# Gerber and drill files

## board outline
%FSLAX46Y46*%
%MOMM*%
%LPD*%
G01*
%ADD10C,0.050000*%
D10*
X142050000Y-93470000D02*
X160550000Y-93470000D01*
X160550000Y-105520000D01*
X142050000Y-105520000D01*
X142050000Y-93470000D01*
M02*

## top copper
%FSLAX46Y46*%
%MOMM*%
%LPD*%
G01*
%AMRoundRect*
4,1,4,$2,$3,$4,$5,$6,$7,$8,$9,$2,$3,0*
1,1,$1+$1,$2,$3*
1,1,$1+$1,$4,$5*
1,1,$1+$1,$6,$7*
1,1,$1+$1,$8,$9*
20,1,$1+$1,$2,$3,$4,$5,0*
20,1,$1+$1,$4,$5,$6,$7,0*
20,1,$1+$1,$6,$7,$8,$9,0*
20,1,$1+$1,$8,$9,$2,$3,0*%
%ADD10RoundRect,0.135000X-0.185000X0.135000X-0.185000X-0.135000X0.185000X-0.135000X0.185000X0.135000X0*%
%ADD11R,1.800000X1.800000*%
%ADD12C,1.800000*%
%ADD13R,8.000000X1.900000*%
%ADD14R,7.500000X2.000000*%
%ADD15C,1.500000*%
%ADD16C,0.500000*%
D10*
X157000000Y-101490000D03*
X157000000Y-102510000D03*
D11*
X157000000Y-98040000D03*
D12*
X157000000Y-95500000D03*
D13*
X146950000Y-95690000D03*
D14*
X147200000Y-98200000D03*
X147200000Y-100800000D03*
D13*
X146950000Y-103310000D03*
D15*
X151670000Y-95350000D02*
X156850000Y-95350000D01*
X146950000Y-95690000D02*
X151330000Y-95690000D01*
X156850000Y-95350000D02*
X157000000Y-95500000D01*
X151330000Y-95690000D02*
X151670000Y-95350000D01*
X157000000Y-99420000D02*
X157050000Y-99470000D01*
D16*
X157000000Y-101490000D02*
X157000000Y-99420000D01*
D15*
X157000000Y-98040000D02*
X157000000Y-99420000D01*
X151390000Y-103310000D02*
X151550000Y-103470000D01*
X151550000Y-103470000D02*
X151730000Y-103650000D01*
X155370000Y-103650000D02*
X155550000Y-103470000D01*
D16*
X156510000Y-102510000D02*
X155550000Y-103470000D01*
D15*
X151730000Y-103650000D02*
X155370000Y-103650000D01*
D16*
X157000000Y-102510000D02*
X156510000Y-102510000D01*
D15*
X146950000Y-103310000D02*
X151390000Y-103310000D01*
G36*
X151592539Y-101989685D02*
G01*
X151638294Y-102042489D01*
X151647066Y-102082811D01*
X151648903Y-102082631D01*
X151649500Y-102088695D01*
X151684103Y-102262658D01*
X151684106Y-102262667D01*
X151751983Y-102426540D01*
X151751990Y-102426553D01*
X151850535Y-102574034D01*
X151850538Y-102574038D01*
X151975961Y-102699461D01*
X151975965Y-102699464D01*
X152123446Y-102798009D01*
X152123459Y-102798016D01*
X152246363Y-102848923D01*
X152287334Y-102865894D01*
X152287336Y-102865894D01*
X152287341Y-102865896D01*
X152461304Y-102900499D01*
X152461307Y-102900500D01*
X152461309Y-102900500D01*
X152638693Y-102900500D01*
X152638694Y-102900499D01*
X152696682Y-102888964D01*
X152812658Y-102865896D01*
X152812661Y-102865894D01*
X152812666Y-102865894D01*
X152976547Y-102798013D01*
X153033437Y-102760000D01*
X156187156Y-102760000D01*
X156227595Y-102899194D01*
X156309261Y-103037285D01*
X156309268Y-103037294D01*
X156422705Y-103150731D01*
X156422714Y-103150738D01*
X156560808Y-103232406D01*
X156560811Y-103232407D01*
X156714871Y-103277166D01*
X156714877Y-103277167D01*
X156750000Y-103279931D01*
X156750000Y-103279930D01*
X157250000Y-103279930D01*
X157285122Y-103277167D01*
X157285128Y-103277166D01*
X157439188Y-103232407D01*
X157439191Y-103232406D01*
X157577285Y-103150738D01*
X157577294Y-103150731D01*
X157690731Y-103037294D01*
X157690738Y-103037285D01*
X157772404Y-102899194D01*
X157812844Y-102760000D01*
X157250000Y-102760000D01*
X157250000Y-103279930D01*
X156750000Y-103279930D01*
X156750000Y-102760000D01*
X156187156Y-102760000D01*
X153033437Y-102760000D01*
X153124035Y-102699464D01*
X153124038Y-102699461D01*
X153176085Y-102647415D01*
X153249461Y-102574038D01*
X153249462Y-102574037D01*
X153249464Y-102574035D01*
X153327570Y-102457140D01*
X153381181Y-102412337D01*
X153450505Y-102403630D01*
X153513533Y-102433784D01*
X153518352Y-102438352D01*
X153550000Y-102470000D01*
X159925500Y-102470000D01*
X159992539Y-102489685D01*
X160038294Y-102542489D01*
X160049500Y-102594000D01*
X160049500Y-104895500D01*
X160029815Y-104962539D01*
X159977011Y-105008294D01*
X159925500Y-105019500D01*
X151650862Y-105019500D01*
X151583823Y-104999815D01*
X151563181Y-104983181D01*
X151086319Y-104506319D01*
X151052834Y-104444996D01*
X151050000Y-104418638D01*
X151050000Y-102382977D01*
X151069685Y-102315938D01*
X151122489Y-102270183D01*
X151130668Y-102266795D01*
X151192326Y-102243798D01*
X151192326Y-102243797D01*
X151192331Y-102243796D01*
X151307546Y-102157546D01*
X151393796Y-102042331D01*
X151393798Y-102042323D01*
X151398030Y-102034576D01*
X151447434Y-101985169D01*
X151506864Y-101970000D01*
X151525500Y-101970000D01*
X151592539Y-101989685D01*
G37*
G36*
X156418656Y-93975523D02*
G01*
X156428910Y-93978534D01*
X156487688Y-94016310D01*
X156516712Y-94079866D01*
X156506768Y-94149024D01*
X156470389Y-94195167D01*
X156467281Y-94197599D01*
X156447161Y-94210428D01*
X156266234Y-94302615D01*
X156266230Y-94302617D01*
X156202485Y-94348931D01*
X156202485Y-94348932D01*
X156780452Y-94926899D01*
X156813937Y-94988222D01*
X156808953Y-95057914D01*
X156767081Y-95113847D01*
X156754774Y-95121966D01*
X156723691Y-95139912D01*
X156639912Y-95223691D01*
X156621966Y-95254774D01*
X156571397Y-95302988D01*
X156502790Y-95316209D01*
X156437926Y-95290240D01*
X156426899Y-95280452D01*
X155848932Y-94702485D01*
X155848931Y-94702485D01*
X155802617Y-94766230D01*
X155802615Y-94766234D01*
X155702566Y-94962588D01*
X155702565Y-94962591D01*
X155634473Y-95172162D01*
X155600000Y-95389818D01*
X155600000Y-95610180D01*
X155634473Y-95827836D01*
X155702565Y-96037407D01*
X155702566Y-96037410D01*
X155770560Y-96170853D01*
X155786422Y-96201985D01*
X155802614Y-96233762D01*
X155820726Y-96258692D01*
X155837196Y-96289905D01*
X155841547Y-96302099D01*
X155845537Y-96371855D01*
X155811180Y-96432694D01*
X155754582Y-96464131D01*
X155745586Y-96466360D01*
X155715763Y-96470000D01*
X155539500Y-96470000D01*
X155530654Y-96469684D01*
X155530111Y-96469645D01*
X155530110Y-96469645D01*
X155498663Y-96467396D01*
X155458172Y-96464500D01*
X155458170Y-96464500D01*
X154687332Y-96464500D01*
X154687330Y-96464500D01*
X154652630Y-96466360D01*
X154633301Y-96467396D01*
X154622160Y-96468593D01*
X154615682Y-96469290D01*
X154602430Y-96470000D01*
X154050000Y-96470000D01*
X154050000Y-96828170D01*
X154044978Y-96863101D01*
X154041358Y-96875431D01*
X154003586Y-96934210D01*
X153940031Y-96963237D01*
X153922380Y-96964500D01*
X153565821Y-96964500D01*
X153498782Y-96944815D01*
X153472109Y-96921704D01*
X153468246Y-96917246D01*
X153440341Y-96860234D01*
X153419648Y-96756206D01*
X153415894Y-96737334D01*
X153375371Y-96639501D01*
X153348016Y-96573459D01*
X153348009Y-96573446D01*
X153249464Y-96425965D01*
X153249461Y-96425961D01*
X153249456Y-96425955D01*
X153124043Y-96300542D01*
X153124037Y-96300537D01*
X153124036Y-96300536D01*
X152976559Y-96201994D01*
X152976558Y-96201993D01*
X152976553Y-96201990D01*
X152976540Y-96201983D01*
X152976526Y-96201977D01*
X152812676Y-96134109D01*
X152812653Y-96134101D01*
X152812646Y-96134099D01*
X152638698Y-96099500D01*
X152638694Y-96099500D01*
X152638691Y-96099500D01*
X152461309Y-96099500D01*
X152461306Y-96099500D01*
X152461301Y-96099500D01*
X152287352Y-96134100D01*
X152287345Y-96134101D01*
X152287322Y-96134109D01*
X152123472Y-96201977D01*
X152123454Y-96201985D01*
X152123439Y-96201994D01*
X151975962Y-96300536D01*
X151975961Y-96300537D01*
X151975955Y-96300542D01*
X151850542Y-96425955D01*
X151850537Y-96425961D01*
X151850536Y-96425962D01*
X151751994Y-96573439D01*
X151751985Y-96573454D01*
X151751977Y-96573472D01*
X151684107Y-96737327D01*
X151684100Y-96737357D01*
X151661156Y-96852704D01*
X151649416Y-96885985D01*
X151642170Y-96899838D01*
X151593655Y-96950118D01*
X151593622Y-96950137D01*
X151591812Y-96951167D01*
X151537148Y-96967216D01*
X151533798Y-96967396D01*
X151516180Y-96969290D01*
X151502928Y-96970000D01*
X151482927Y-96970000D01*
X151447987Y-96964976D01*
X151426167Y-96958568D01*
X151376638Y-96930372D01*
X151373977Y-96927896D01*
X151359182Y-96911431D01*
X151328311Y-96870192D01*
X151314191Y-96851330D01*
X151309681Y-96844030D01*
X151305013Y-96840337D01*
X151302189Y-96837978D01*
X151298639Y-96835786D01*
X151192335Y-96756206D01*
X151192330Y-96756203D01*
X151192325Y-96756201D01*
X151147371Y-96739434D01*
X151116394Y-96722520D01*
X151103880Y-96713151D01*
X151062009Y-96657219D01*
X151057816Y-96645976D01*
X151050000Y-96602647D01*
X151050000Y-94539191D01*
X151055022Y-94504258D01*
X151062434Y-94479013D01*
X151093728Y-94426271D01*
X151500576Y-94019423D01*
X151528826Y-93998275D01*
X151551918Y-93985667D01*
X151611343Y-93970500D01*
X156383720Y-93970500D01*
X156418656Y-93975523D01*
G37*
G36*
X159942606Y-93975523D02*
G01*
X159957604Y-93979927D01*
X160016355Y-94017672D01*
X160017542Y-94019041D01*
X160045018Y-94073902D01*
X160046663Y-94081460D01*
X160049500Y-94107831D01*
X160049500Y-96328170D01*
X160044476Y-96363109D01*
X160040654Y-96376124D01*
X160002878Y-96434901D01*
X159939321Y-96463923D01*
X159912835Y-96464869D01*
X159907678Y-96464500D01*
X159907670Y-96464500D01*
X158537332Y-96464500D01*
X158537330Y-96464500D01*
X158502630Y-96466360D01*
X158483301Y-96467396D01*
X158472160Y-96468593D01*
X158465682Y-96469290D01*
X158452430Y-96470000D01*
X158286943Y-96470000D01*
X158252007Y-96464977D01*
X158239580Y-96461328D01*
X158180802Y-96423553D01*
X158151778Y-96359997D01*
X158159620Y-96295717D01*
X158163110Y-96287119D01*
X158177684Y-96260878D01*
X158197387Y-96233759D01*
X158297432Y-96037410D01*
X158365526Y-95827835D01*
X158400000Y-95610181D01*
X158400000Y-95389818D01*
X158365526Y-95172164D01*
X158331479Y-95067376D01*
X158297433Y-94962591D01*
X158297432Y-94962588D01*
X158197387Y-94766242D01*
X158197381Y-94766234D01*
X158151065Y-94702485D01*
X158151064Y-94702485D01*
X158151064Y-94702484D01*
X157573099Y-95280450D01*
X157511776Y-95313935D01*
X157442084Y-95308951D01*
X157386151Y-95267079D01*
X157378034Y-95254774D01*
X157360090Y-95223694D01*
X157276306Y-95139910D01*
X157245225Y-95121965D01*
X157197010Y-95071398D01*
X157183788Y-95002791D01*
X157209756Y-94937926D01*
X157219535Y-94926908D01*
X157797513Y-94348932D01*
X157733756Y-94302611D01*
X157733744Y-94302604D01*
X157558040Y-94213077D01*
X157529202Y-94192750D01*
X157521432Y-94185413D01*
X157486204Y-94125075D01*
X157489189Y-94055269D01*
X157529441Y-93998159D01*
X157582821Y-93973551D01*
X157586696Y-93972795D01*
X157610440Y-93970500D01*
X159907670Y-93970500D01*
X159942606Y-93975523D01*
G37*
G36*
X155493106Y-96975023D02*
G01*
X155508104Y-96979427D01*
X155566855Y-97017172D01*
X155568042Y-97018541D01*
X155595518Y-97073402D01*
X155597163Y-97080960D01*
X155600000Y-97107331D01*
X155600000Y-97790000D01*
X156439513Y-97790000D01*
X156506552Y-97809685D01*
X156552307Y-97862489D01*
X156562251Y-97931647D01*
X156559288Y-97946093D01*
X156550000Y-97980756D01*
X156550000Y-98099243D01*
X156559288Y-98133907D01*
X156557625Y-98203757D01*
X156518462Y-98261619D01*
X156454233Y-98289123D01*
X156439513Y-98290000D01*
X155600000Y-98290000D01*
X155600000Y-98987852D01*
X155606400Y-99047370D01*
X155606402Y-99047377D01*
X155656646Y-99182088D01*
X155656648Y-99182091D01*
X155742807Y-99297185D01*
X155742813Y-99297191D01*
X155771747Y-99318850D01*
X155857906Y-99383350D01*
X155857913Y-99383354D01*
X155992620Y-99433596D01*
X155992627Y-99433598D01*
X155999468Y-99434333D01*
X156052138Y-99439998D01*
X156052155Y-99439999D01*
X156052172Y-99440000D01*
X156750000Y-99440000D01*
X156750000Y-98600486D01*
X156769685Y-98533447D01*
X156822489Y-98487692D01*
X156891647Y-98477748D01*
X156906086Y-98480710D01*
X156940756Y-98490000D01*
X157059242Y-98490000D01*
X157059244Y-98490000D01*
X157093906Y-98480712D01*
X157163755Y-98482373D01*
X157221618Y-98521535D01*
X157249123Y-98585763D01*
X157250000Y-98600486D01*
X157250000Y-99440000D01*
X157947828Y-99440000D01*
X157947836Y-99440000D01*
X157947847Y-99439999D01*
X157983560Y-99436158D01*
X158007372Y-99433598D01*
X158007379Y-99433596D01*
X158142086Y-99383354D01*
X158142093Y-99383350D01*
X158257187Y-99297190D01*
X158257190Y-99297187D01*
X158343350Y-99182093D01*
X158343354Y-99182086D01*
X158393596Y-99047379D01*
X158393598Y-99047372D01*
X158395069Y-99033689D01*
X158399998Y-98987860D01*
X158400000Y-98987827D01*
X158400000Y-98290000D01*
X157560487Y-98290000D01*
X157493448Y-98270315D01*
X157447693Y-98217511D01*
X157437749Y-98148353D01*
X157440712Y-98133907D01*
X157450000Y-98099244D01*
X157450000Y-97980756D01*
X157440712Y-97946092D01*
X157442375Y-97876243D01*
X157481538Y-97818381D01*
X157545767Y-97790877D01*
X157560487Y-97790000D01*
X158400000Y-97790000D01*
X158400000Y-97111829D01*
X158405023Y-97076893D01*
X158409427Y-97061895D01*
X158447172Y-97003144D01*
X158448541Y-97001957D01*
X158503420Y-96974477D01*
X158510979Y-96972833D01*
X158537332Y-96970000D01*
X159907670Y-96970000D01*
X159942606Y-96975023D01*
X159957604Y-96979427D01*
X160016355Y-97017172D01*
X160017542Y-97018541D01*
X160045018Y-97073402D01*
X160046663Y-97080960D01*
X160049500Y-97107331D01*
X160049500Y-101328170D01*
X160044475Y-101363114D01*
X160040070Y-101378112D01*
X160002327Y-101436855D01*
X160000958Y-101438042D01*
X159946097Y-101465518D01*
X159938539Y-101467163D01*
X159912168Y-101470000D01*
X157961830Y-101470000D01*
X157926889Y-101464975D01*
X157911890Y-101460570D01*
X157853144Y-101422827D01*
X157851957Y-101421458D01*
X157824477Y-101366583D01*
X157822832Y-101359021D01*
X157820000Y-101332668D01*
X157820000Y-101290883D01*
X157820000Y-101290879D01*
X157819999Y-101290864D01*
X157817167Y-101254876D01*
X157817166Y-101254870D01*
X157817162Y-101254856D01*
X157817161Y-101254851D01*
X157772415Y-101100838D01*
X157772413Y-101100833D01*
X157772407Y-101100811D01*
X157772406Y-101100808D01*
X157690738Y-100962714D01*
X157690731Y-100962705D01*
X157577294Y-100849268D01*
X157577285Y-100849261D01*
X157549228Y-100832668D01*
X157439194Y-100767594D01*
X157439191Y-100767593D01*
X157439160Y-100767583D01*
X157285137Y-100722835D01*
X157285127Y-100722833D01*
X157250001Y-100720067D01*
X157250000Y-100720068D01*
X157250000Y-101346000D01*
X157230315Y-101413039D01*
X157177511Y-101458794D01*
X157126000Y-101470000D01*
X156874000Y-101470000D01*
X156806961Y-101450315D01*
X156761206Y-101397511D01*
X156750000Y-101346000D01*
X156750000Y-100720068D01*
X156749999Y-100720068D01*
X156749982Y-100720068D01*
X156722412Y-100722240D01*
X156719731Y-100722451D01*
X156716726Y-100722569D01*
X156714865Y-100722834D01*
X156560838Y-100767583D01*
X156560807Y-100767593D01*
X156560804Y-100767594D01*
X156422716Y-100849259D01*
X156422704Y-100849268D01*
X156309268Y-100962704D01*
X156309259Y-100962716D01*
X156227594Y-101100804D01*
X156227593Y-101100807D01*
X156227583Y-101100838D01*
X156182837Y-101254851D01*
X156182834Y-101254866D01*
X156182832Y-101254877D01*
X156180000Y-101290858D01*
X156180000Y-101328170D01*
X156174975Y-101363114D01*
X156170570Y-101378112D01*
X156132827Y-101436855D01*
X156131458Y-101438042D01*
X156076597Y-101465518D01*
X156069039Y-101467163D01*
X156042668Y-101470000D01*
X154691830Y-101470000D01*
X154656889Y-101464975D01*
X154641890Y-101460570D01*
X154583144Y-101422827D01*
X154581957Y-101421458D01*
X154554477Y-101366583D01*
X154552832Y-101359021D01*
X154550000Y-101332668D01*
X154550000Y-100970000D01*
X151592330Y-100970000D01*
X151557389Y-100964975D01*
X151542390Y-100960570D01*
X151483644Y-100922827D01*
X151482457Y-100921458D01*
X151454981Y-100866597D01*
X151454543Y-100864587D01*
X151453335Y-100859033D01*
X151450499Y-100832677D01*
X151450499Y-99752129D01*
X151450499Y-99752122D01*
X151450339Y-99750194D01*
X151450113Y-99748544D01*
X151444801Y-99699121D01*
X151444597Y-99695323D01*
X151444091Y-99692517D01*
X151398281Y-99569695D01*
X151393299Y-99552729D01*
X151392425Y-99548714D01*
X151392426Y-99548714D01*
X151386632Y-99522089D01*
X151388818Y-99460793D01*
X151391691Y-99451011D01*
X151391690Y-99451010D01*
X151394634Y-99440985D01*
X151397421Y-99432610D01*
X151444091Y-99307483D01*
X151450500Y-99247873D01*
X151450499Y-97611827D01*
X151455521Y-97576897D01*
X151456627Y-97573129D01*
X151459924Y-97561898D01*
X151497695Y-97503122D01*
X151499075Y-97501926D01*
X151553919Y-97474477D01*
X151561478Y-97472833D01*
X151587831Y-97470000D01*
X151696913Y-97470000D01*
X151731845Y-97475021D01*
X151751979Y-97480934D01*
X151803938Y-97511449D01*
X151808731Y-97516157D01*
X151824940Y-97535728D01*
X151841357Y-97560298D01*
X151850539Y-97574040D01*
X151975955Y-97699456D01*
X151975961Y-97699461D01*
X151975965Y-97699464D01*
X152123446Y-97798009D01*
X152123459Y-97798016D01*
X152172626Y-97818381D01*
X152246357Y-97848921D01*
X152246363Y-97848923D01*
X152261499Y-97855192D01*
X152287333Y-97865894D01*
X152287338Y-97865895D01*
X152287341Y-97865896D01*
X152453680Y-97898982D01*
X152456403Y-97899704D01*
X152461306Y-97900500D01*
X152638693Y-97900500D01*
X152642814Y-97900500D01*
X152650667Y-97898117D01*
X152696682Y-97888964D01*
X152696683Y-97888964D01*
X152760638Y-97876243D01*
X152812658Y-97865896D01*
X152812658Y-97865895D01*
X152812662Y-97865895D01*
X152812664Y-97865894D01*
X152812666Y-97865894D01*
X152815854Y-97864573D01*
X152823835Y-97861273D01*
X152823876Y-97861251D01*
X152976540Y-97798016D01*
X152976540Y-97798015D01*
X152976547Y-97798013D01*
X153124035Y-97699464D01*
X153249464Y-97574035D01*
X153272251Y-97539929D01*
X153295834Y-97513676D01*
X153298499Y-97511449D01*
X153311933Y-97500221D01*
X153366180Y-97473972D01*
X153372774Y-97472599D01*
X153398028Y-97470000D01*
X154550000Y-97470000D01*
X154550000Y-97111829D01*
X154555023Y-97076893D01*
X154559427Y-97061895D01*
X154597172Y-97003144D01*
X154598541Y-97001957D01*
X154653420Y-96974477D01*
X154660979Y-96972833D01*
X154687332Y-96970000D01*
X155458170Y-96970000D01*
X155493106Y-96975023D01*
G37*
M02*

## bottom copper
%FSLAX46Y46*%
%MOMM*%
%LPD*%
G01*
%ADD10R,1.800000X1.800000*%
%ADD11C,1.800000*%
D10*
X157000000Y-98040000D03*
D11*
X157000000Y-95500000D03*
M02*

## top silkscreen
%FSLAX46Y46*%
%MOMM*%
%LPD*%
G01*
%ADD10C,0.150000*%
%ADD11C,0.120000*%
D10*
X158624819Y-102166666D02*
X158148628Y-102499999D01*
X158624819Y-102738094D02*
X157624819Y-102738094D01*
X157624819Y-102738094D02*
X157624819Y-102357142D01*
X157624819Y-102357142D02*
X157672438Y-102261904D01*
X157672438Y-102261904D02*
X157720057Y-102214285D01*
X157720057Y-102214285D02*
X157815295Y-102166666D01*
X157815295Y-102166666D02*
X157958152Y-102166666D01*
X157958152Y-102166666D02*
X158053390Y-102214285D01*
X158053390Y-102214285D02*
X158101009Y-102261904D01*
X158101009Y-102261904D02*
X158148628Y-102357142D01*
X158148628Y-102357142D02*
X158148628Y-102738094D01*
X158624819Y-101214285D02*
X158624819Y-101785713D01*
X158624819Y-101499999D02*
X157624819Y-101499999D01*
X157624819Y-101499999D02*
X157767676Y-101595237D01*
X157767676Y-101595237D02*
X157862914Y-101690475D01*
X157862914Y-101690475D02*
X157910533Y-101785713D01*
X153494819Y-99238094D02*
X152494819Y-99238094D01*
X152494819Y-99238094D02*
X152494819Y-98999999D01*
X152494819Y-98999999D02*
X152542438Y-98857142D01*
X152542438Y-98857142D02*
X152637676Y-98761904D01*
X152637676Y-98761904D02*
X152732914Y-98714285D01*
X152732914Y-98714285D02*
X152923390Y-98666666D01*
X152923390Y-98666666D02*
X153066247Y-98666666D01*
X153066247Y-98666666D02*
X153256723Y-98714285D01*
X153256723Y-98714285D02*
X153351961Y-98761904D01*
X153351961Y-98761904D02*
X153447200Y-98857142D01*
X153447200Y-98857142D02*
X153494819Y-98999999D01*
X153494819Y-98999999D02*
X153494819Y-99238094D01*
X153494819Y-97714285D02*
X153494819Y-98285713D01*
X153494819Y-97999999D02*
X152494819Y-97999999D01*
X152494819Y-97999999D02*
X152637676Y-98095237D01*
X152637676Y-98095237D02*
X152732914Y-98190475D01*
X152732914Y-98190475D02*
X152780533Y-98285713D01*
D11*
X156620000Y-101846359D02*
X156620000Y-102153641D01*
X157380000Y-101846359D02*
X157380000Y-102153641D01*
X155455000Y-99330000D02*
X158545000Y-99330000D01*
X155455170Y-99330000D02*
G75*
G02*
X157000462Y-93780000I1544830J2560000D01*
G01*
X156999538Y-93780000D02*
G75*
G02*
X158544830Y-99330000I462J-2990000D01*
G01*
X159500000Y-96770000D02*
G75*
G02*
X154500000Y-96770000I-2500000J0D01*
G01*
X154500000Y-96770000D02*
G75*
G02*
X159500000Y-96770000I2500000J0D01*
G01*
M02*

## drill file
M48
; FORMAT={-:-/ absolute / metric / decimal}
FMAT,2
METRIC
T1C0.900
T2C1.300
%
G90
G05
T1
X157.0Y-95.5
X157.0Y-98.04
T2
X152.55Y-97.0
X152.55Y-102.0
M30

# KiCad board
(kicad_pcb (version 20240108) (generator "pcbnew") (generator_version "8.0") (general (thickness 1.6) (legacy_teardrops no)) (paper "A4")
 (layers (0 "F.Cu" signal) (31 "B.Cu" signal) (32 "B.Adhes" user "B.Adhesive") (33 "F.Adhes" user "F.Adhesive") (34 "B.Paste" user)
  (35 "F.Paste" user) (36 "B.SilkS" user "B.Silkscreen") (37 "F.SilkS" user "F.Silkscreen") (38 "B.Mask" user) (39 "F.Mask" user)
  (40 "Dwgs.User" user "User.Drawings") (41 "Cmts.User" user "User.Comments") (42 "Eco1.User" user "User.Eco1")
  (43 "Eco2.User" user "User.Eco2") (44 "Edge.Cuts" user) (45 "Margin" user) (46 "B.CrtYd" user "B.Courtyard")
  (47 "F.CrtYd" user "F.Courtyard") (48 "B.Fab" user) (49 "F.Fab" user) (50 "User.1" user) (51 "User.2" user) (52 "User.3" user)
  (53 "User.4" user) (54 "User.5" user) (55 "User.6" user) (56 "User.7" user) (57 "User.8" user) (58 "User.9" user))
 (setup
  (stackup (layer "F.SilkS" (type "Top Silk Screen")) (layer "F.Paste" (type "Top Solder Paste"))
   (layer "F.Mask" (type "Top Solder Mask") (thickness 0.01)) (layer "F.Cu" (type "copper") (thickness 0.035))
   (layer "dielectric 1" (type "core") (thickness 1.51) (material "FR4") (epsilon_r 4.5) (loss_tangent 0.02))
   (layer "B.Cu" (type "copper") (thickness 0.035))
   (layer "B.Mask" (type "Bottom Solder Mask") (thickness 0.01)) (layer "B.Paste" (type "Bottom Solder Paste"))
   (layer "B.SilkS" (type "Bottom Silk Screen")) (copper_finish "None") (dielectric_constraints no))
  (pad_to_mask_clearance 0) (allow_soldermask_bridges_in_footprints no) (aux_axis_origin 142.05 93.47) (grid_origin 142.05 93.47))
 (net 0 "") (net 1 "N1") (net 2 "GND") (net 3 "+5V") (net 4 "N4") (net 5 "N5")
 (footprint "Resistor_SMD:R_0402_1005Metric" (layer "F.Cu") (at 157 102 -90)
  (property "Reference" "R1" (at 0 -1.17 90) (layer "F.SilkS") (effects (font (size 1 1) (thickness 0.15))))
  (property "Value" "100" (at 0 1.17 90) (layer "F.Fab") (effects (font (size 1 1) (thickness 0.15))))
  (fp_line (start -0.153641 0.38) (end 0.153641 0.38) (stroke (width 0.12) (type solid)) (layer "F.SilkS"))
  (fp_line (start -0.153641 -0.38) (end 0.153641 -0.38) (stroke (width 0.12) (type solid)) (layer "F.SilkS"))
  (pad "1" smd roundrect (at -0.51 0 270) (size 0.54 0.64) (layers "F.Cu" "F.Paste" "F.Mask") (roundrect_rratio 0.25) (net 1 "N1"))
  (pad "2" smd roundrect (at 0.51 0 270) (size 0.54 0.64) (layers "F.Cu" "F.Paste" "F.Mask") (roundrect_rratio 0.25) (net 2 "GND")))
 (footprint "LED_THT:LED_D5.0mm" (layer "F.Cu") (at 157 98.04 90)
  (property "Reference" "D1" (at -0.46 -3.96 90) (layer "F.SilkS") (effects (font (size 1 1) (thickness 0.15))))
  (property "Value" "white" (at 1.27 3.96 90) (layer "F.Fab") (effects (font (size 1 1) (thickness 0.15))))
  (fp_line (start -1.29 -1.545) (end -1.29 1.545) (stroke (width 0.12) (type solid)) (layer "F.SilkS"))
  (fp_arc (start -1.29 -1.54483) (mid 2.072002 -2.880433) (end 4.26 0.000462) (stroke (width 0.12) (type solid)) (layer "F.SilkS"))
  (fp_arc (start 4.26 -0.000462) (mid 2.072002 2.880433) (end -1.29 1.54483) (stroke (width 0.12) (type solid)) (layer "F.SilkS"))
  (fp_circle (center 1.27 0) (end 3.77 0) (stroke (width 0.12) (type solid)) (fill none) (layer "F.SilkS"))
  (pad "1" thru_hole rect (at 0 0 90) (size 1.8 1.8) (drill 0.9) (layers "*.Cu" "*.Mask") (remove_unused_layers no) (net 1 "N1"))
  (pad "2" thru_hole circle (at 2.54 0 90) (size 1.8 1.8) (drill 0.9) (layers "*.Cu" "*.Mask") (remove_unused_layers no) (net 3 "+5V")))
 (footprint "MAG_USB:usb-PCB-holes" (layer "F.Cu") (at 142.05 99.5 -90)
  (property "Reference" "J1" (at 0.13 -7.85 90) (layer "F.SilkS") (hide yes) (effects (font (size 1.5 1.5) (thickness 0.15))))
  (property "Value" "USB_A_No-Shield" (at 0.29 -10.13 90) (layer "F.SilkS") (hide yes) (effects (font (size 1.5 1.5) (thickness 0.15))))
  (pad "" np_thru_hole circle (at -2.5 -10.5 270) (size 1.3 1.3) (drill 1.3) (layers "F&B.Cu" "*.Mask"))
  (pad "" np_thru_hole circle (at 2.5 -10.5 270) (size 1.3 1.3) (drill 1.3) (layers "F&B.Cu" "*.Mask"))
  (pad "1" connect rect (at -3.81 -4.9 270) (size 1.9 8) (layers "F.Cu" "F.Mask") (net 3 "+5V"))
  (pad "2" connect rect (at -1.3 -5.15 270) (size 2 7.5) (layers "F.Cu" "F.Mask") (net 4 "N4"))
  (pad "3" connect rect (at 1.3 -5.15 270) (size 2 7.5) (layers "F.Cu" "F.Mask") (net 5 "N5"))
  (pad "4" connect rect (at 3.81 -4.9 270) (size 1.9 8) (layers "F.Cu" "F.Mask") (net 2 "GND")))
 (gr_rect (start 142.05 93.47) (end 160.55 105.52) (stroke (width 0.05) (type default)) (fill none) (layer "Edge.Cuts"))
 (segment (start 151.67 95.35) (end 156.85 95.35) (width 1.5) (layer "F.Cu") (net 3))
 (segment (start 146.95 95.69) (end 151.33 95.69) (width 1.5) (layer "F.Cu") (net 3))
 (segment (start 156.85 95.35) (end 157 95.5) (width 1.5) (layer "F.Cu") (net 3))
 (segment (start 151.33 95.69) (end 151.67 95.35) (width 1.5) (layer "F.Cu") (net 3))
 (segment (start 157 99.42) (end 157.05 99.47) (width 1.5) (layer "F.Cu") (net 1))
 (segment (start 157 101.49) (end 157 99.42) (width 0.5) (layer "F.Cu") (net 1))
 (segment (start 157 98.04) (end 157 99.42) (width 1.5) (layer "F.Cu") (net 1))
 (segment (start 151.39 103.31) (end 151.55 103.47) (width 1.5) (layer "F.Cu") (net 2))
 (segment (start 151.55 103.47) (end 151.73 103.65) (width 1.5) (layer "F.Cu") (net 2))
 (segment (start 155.37 103.65) (end 155.55 103.47) (width 1.5) (layer "F.Cu") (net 2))
 (segment (start 156.51 102.51) (end 155.55 103.47) (width 0.5) (layer "F.Cu") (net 2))
 (segment (start 151.73 103.65) (end 155.37 103.65) (width 1.5) (layer "F.Cu") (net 2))
 (segment (start 157 102.51) (end 156.51 102.51) (width 0.5) (layer "F.Cu") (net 2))
 (segment (start 146.95 103.31) (end 151.39 103.31) (width 1.5) (layer "F.Cu") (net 2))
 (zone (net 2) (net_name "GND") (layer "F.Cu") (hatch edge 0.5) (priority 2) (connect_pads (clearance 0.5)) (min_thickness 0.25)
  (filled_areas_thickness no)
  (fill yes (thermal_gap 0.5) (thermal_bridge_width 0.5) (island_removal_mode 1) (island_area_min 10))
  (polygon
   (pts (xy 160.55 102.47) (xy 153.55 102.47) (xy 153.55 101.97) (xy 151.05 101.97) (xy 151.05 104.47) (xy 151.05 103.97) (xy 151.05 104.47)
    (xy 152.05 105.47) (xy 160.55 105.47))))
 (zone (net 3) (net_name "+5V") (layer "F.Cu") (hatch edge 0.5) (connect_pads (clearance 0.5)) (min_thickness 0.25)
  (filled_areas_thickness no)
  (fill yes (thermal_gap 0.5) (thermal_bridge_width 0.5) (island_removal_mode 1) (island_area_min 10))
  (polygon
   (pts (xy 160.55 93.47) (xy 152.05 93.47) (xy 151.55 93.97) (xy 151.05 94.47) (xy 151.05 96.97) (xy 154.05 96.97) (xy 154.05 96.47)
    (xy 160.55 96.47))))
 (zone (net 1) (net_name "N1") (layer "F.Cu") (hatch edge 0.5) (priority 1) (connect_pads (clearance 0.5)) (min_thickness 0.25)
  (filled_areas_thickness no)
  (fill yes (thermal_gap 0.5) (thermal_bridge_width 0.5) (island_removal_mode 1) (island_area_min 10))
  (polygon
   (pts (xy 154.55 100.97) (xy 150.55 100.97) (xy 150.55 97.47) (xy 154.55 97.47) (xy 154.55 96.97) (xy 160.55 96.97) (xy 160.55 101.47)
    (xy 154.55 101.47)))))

